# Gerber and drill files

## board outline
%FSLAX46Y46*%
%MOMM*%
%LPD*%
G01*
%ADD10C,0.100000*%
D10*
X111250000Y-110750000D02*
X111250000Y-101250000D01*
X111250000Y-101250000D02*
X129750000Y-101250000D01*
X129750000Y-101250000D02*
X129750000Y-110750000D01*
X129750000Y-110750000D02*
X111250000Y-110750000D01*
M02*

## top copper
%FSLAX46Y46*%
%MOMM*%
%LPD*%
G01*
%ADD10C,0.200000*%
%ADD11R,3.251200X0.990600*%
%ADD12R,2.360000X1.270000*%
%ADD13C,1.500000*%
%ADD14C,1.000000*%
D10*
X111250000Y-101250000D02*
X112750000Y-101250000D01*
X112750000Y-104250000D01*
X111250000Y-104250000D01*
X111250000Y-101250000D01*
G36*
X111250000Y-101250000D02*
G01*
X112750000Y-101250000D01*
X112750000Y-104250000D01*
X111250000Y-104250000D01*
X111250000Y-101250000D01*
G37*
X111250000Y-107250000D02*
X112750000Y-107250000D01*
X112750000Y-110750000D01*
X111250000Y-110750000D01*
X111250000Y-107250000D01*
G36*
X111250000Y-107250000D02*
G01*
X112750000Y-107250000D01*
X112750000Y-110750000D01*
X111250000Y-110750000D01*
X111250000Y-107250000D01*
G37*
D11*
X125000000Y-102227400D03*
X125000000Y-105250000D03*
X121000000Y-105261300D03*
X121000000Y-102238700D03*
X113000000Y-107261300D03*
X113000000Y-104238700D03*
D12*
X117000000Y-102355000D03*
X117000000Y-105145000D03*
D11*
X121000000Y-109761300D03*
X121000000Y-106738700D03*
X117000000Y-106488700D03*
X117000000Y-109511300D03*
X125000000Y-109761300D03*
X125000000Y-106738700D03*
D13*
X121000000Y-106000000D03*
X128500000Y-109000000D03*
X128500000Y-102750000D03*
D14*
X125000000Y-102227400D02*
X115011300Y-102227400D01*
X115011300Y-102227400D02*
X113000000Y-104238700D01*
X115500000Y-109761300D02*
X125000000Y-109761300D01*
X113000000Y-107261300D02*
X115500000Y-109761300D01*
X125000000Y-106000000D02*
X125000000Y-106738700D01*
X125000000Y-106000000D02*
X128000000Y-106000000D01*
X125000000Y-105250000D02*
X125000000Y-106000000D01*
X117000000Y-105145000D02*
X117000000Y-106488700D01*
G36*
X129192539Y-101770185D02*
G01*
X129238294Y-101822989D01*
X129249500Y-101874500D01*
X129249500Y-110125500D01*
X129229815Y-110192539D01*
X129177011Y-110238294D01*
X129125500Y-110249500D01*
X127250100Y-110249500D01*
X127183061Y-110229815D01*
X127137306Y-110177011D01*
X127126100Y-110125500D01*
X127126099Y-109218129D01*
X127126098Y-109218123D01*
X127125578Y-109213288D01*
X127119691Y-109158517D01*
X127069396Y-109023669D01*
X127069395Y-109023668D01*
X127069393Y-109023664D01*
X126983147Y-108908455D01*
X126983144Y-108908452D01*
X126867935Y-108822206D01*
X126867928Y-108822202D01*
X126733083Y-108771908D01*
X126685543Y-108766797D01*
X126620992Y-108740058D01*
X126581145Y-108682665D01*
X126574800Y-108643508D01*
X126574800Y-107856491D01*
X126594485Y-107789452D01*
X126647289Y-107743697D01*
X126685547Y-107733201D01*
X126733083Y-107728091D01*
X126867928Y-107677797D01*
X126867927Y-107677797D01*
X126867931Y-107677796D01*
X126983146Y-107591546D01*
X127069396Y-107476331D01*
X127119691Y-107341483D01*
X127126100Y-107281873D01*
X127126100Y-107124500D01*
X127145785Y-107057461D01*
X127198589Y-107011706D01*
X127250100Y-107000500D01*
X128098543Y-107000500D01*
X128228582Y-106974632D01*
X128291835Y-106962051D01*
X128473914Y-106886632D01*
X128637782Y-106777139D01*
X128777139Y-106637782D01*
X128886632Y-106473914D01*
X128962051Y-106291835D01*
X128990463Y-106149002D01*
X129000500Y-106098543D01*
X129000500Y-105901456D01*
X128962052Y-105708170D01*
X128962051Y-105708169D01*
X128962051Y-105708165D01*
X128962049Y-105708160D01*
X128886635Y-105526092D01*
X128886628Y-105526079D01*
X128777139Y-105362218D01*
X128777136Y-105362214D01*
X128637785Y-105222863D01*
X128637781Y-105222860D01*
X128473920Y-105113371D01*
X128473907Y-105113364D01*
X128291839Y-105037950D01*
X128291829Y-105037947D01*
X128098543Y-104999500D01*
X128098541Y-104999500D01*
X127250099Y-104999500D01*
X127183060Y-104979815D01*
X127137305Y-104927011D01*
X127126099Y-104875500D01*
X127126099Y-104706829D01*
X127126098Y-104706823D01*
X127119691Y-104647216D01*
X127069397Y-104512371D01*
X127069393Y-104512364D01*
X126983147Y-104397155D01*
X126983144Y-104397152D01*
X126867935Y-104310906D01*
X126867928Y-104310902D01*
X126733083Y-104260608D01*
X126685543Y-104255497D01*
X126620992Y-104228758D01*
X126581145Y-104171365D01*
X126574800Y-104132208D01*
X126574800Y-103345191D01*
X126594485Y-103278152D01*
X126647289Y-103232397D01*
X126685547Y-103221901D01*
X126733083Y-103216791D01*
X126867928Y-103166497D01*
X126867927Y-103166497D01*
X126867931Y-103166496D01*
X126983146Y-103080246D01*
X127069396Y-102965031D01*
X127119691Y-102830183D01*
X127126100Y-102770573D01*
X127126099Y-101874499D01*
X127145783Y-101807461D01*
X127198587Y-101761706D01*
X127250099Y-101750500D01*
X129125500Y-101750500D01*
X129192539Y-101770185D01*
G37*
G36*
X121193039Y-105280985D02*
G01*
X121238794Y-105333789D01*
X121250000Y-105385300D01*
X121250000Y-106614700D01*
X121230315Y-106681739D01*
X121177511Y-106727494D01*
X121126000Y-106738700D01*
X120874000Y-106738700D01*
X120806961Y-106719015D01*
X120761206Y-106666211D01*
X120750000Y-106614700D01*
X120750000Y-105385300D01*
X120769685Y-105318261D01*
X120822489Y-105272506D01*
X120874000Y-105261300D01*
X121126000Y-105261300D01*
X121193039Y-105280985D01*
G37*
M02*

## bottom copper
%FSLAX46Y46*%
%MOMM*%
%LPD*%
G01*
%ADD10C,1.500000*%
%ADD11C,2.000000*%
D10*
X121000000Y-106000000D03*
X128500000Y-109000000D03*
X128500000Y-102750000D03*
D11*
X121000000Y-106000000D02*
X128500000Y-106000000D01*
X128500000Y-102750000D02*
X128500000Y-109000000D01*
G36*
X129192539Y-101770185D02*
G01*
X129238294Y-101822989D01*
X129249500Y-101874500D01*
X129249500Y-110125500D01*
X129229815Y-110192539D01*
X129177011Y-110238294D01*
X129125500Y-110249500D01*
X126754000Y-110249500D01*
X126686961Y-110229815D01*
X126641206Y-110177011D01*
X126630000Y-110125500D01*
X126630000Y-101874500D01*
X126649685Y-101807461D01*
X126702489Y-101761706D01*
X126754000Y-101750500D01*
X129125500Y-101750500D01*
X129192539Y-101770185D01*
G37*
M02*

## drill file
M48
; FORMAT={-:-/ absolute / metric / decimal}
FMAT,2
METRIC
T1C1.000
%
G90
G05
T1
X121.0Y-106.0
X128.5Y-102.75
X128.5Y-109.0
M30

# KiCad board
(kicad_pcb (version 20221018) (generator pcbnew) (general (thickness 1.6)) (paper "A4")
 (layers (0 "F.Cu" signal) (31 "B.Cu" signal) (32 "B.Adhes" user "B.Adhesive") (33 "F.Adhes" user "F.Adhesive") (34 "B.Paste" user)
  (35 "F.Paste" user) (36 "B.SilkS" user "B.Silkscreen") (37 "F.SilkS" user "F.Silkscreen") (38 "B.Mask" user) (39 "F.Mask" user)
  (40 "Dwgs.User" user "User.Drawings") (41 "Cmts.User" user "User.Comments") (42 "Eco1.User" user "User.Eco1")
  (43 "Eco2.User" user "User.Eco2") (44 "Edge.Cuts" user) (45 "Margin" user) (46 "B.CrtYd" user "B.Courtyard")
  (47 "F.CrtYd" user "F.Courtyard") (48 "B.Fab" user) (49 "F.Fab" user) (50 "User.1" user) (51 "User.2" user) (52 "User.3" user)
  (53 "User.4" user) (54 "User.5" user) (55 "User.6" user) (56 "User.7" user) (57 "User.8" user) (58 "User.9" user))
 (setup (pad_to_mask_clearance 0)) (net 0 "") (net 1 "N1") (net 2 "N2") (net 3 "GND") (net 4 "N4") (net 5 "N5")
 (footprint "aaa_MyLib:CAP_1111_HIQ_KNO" (layer "F.Cu") (at 125 103.7387 -90)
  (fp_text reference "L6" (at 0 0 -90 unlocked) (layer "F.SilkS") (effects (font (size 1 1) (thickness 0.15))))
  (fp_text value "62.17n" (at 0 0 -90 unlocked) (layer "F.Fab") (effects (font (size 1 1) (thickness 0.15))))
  (pad "1" smd rect (at -1.5113 0 270) (size 0.9906 3.2512) (layers "F.Cu" "F.Paste" "F.Mask") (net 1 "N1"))
  (pad "2" smd rect (at 1.5113 0 270) (size 0.9906 3.2512) (layers "F.Cu" "F.Paste" "F.Mask") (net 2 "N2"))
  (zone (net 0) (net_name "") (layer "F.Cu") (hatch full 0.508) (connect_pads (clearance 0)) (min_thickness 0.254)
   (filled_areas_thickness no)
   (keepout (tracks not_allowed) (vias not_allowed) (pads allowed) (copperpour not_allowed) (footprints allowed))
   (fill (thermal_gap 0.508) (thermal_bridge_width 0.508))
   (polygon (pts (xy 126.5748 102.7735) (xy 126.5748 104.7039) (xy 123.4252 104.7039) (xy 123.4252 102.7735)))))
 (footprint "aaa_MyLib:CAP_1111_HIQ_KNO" (layer "F.Cu") (at 121 103.75 90)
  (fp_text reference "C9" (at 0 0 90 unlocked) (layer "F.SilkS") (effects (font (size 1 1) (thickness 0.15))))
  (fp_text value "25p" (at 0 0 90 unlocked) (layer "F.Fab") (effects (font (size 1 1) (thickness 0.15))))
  (pad "1" smd rect (at -1.5113 0 90) (size 0.9906 3.2512) (layers "F.Cu" "F.Paste" "F.Mask") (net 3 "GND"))
  (pad "2" smd rect (at 1.5113 0 90) (size 0.9906 3.2512) (layers "F.Cu" "F.Paste" "F.Mask") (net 1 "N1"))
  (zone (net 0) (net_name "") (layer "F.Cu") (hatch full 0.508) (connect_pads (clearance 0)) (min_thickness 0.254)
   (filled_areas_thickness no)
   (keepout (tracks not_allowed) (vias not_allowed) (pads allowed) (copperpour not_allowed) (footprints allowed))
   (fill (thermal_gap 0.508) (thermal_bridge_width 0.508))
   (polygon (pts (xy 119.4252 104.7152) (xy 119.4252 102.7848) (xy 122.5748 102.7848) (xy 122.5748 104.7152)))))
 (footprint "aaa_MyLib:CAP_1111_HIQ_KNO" (layer "F.Cu") (at 113 105.75 90)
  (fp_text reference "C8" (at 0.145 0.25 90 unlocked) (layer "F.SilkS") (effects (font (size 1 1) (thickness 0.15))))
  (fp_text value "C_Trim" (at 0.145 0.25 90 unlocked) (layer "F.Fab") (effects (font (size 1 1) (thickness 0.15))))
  (pad "1" smd rect (at -1.5113 0 90) (size 0.9906 3.2512) (layers "F.Cu" "F.Paste" "F.Mask") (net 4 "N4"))
  (pad "2" smd rect (at 1.5113 0 90) (size 0.9906 3.2512) (layers "F.Cu" "F.Paste" "F.Mask") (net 1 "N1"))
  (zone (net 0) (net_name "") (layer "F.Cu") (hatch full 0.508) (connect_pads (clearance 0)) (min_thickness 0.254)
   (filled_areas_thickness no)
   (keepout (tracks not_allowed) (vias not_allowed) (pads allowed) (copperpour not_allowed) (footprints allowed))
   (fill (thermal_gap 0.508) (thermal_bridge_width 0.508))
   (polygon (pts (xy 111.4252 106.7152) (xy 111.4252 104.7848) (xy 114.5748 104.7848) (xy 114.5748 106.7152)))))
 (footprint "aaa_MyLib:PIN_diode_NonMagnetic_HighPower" (layer "F.Cu") (at 117 103.75 -90)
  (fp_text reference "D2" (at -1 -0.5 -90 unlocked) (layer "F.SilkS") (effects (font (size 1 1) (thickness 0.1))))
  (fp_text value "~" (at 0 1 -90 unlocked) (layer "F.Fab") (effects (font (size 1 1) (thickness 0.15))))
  (pad "1" smd rect (at -1.395 0 270) (size 1.27 2.36) (layers "F.Cu" "F.Paste" "F.Mask") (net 1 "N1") (thermal_bridge_angle 45))
  (pad "2" smd rect (at 1.395 0 270) (size 1.27 2.36) (layers "F.Cu" "F.Paste" "F.Mask") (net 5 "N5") (thermal_bridge_angle 45))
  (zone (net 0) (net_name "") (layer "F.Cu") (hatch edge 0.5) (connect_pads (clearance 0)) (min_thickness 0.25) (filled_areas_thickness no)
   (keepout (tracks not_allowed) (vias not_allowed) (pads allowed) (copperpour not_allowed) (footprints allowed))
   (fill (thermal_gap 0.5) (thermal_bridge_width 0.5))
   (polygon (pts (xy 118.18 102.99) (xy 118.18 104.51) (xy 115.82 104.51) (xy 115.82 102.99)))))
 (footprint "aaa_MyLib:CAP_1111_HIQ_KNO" (layer "F.Cu") (at 121 108.25 90)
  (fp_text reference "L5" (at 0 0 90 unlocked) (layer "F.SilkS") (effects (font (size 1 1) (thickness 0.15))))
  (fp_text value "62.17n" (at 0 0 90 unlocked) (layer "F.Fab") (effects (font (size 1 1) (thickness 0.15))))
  (pad "1" smd rect (at -1.5113 0 90) (size 0.9906 3.2512) (layers "F.Cu" "F.Paste" "F.Mask") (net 4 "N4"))
  (pad "2" smd rect (at 1.5113 0 90) (size 0.9906 3.2512) (layers "F.Cu" "F.Paste" "F.Mask") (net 3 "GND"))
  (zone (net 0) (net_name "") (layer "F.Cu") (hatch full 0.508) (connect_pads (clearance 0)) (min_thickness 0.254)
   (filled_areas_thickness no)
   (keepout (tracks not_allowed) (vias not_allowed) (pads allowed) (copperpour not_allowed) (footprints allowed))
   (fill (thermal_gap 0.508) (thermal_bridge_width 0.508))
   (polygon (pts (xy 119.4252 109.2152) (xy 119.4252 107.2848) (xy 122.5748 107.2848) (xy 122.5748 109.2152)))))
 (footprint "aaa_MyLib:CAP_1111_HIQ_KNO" (layer "F.Cu") (at 117 108 -90)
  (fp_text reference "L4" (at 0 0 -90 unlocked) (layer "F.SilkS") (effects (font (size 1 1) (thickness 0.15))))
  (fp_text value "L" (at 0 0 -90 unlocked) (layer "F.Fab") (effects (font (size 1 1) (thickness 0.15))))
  (pad "1" smd rect (at -1.5113 0 270) (size 0.9906 3.2512) (layers "F.Cu" "F.Paste" "F.Mask") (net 5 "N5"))
  (pad "2" smd rect (at 1.5113 0 270) (size 0.9906 3.2512) (layers "F.Cu" "F.Paste" "F.Mask") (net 4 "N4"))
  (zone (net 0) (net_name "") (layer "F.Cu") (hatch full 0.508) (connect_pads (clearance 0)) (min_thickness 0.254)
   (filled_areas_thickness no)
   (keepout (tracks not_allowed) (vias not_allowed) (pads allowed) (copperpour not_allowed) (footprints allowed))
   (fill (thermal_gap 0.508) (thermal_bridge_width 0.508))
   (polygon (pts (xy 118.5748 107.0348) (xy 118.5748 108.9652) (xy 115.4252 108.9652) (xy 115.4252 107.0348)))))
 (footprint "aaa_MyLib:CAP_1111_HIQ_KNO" (layer "F.Cu") (at 125 108.25 90)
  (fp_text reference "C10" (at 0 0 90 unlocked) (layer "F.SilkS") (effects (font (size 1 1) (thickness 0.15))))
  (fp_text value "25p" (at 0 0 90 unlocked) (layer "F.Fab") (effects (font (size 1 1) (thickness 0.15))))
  (pad "1" smd rect (at -1.5113 0 90) (size 0.9906 3.2512) (layers "F.Cu" "F.Paste" "F.Mask") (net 4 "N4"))
  (pad "2" smd rect (at 1.5113 0 90) (size 0.9906 3.2512) (layers "F.Cu" "F.Paste" "F.Mask") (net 2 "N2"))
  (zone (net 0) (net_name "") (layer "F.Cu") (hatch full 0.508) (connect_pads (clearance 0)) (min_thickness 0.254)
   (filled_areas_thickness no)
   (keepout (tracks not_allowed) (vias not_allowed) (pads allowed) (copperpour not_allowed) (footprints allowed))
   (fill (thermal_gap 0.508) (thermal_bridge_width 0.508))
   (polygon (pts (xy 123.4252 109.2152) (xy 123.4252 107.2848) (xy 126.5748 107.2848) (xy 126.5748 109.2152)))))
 (gr_rect (start 111.25 101.25) (end 112.75 104.25) (stroke (width 0.2) (type solid)) (fill solid) (layer "F.Cu"))
 (gr_rect (start 111.25 107.25) (end 112.75 110.75) (stroke (width 0.2) (type solid)) (fill solid) (layer "F.Cu"))
 (gr_line (start 111.25 110.75) (end 111.25 101.25) (stroke (width 0.1) (type default)) (layer "Edge.Cuts"))
 (gr_line (start 111.25 101.25) (end 129.75 101.25) (stroke (width 0.1) (type default)) (layer "Edge.Cuts"))
 (gr_line (start 129.75 101.25) (end 129.75 110.75) (stroke (width 0.1) (type default)) (layer "Edge.Cuts"))
 (gr_line (start 129.75 110.75) (end 111.25 110.75) (stroke (width 0.1) (type default)) (layer "Edge.Cuts"))
 (via (at 121 106) (size 1.5) (drill 1) (layers "F.Cu" "B.Cu") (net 3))
 (via (at 128.5 109) (size 1.5) (drill 1) (layers "F.Cu" "B.Cu") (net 3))
 (via (at 128.5 102.75) (size 1.5) (drill 1) (layers "F.Cu" "B.Cu") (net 3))
 (segment (start 121 106) (end 128.5 106) (width 2) (layer "B.Cu") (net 3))
 (segment (start 128.5 102.75) (end 128.5 109) (width 2) (layer "B.Cu") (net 3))
 (segment (start 125 102.2274) (end 115.0113 102.2274) (width 1) (layer "F.Cu") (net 1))
 (segment (start 115.0113 102.2274) (end 113 104.2387) (width 1) (layer "F.Cu") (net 1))
 (segment (start 115.5 109.7613) (end 125 109.7613) (width 1) (layer "F.Cu") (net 4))
 (segment (start 113 107.2613) (end 115.5 109.7613) (width 1) (layer "F.Cu") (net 4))
 (segment (start 125 106) (end 125 106.7387) (width 1) (layer "F.Cu") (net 2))
 (segment (start 125 106) (end 128 106) (width 1) (layer "F.Cu") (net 2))
 (segment (start 125 105.25) (end 125 106) (width 1) (layer "F.Cu") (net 2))
 (segment (start 117 105.145) (end 117 106.4887) (width 1) (layer "F.Cu") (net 5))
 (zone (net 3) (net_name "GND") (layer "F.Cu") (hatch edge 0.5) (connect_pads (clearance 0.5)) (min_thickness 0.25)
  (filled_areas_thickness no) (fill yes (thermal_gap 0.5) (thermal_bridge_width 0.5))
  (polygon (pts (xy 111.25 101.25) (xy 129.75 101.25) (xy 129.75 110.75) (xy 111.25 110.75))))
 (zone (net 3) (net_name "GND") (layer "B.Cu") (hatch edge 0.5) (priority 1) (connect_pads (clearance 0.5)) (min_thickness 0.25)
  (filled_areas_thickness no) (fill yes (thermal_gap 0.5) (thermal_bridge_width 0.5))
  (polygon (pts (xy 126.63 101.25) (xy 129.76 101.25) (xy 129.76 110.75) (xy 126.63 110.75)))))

